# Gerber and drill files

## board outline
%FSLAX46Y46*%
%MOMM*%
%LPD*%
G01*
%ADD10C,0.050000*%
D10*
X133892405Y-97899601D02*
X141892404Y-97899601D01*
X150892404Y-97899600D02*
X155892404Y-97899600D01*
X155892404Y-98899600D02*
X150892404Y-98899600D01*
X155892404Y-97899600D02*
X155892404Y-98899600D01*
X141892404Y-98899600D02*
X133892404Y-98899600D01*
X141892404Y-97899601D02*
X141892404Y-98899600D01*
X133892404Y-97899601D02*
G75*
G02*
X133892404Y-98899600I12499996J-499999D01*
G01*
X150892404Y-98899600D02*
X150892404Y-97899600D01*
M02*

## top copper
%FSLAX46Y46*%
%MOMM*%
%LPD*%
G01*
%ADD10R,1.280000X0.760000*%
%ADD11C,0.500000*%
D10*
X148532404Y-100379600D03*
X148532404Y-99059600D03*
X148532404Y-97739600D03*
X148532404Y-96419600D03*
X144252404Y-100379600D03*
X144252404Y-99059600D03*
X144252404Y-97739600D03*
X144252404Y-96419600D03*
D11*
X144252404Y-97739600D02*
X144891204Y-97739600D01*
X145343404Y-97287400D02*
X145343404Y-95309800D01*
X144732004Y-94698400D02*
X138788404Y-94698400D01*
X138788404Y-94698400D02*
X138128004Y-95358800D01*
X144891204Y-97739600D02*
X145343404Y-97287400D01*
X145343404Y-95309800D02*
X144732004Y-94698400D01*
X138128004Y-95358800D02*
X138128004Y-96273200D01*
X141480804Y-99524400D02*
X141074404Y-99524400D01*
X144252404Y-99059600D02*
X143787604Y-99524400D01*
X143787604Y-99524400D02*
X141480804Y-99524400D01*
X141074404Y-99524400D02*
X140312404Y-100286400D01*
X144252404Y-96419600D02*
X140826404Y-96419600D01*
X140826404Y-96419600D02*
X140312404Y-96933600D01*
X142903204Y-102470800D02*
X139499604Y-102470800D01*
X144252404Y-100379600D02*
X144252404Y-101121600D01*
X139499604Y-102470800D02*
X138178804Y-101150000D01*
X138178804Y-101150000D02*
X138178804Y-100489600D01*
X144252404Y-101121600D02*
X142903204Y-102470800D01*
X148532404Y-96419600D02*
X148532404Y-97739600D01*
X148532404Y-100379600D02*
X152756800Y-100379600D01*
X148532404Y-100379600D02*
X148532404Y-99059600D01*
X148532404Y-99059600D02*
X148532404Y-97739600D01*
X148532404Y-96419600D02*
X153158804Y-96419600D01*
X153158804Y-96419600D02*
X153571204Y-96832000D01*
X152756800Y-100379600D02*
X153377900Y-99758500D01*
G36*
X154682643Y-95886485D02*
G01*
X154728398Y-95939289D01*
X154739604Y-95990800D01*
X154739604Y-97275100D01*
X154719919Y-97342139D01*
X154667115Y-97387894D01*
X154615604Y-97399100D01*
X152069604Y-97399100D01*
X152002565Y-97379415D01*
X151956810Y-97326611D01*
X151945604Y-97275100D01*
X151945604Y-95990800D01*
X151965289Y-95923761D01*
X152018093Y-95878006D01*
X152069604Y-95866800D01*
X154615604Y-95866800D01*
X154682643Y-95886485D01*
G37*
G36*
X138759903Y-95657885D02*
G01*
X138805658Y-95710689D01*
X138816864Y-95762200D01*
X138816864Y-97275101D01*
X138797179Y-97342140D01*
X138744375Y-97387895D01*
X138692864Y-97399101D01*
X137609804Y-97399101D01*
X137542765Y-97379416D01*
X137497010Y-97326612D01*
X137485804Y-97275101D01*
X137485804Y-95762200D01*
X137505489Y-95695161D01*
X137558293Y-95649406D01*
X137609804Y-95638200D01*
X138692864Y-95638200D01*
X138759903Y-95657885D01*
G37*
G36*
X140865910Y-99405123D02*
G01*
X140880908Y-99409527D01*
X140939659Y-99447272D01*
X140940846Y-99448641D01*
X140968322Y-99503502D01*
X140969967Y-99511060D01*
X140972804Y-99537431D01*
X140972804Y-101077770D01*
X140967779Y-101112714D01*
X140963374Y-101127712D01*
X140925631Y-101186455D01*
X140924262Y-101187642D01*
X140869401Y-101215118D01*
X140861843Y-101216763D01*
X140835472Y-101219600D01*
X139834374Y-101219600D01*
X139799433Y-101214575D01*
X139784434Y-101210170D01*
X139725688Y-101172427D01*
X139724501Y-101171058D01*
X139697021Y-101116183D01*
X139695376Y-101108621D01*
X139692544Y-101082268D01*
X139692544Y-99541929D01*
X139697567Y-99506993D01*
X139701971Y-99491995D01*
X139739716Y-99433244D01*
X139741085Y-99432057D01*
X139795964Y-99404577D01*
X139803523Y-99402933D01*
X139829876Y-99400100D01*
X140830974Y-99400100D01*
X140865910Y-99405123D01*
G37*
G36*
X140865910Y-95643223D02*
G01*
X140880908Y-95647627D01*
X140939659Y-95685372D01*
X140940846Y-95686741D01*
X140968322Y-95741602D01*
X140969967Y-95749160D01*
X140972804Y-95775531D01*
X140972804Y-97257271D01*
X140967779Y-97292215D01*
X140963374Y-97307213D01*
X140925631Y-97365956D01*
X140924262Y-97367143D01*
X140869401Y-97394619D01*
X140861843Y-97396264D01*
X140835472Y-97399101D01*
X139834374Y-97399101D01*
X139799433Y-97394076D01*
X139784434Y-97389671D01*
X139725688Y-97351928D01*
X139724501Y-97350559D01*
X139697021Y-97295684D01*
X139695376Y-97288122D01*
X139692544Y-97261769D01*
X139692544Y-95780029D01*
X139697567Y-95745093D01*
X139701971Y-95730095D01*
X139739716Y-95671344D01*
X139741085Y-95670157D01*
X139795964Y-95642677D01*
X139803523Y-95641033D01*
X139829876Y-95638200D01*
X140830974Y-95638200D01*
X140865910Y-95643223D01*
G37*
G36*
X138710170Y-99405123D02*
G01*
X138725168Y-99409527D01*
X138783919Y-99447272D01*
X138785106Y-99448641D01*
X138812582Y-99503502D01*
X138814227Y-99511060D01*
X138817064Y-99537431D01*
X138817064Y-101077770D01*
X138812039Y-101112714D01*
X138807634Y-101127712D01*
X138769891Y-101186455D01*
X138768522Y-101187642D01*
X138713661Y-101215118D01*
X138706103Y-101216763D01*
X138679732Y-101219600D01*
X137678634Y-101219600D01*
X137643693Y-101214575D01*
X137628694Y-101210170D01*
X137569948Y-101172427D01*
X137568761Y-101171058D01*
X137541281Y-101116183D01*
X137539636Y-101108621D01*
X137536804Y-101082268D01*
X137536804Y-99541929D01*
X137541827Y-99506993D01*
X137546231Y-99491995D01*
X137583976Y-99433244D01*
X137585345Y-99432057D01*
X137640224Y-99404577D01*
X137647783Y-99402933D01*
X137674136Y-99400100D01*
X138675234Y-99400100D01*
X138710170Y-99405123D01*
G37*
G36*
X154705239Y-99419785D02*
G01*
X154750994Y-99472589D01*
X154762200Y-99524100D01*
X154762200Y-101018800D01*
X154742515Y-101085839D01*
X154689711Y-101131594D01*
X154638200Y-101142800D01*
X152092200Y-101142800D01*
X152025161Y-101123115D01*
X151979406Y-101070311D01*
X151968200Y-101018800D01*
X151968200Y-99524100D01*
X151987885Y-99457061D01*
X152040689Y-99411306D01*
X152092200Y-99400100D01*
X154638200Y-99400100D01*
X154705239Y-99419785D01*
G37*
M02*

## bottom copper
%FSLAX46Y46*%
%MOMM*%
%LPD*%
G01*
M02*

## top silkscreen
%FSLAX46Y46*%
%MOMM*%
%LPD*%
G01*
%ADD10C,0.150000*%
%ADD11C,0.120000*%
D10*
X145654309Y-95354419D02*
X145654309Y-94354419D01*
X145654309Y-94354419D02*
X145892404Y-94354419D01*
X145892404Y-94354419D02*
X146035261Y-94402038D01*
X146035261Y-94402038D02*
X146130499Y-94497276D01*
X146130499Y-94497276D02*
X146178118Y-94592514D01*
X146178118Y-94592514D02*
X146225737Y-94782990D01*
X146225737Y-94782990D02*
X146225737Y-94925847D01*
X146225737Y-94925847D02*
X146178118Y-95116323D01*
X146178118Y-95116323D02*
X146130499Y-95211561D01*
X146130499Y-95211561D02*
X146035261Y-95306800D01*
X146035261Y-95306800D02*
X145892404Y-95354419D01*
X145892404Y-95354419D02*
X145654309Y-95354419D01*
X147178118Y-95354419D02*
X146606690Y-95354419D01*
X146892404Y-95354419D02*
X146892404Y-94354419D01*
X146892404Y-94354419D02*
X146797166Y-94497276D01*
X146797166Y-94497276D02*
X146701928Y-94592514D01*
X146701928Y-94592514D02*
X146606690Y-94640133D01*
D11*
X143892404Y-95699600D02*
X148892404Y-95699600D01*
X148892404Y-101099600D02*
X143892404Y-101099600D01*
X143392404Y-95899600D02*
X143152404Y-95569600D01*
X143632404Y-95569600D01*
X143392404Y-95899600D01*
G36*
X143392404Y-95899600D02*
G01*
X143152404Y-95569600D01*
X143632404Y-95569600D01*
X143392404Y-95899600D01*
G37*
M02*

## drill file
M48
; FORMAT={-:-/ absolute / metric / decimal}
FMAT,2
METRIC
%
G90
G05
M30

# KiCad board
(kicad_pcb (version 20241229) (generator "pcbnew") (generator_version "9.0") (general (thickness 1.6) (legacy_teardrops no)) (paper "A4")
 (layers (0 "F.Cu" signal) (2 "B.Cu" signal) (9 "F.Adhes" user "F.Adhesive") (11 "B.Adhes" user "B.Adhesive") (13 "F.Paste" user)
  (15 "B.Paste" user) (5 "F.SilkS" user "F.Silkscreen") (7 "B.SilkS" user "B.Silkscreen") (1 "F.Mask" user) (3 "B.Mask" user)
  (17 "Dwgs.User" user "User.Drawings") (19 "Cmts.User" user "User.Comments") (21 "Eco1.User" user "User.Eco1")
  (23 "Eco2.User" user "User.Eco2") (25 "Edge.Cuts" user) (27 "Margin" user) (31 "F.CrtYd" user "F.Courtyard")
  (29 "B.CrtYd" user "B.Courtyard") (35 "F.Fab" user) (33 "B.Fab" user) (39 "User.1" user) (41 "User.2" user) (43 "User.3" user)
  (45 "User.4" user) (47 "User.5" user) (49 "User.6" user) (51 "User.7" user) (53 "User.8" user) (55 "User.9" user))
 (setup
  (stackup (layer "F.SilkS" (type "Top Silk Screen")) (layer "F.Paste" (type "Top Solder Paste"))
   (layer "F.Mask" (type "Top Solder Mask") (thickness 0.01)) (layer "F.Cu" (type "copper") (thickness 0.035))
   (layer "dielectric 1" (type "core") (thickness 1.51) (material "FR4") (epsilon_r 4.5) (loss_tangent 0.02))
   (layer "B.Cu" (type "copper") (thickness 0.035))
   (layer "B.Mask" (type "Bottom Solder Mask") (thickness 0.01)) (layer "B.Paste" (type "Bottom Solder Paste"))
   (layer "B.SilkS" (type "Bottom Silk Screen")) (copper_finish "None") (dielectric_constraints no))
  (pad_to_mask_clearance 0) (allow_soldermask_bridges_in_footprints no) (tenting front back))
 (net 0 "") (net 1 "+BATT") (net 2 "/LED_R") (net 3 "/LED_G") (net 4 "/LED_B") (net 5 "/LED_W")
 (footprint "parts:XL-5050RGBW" (layer "F.Cu") (at 146.392404 98.3996 180)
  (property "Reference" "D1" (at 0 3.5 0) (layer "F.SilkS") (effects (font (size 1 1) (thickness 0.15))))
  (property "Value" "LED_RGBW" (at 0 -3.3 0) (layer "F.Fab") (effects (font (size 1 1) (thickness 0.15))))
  (fp_line (start 2.5 2.7) (end -2.5 2.7) (stroke (width 0.12) (type solid)) (layer "F.SilkS"))
  (fp_line (start -2.5 -2.7) (end 2.5 -2.7) (stroke (width 0.12) (type solid)) (layer "F.SilkS"))
  (fp_poly (pts (xy 3 2.5) (xy 3.24 2.83) (xy 2.76 2.83) (xy 3 2.5)) (stroke (width 0.12) (type solid)) (fill yes) (layer "F.SilkS"))
  (pad "1" smd rect (at -2.14 -1.98 270) (size 0.76 1.28) (layers "F.Cu" "F.Mask" "F.Paste") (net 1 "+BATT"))
  (pad "2" smd rect (at -2.14 -0.66 270) (size 0.76 1.28) (layers "F.Cu" "F.Mask" "F.Paste") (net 1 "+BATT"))
  (pad "3" smd rect (at -2.14 0.66 270) (size 0.76 1.28) (layers "F.Cu" "F.Mask" "F.Paste") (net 1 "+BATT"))
  (pad "4" smd rect (at -2.14 1.98 270) (size 0.76 1.28) (layers "F.Cu" "F.Mask" "F.Paste") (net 1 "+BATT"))
  (pad "5" smd rect (at 2.14 -1.98 270) (size 0.76 1.28) (layers "F.Cu" "F.Mask" "F.Paste") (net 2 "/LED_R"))
  (pad "6" smd rect (at 2.14 -0.66 270) (size 0.76 1.28) (layers "F.Cu" "F.Mask" "F.Paste") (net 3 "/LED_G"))
  (pad "7" smd rect (at 2.14 0.66 270) (size 0.76 1.28) (layers "F.Cu" "F.Mask" "F.Paste") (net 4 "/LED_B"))
  (pad "8" smd rect (at 2.14 1.98 270) (size 0.76 1.28) (layers "F.Cu" "F.Mask" "F.Paste") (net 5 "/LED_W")))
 (gr_line (start 133.892405 97.899601) (end 141.892404 97.899601) (stroke (width 0.05) (type default)) (layer "Edge.Cuts"))
 (gr_line (start 150.892404 97.8996) (end 155.892404 97.8996) (stroke (width 0.05) (type default)) (layer "Edge.Cuts"))
 (gr_line (start 155.892404 98.8996) (end 150.892404 98.8996) (stroke (width 0.05) (type default)) (layer "Edge.Cuts"))
 (gr_line (start 155.892404 97.8996) (end 155.892404 98.8996) (stroke (width 0.05) (type default)) (layer "Edge.Cuts"))
 (gr_line (start 141.892404 98.8996) (end 133.892404 98.8996) (stroke (width 0.05) (type default)) (layer "Edge.Cuts"))
 (gr_line (start 141.892404 97.899601) (end 141.892404 98.8996) (stroke (width 0.05) (type default)) (layer "Edge.Cuts"))
 (gr_arc (start 133.892404 97.899601) (mid 158.9024 98.3996) (end 133.892404 98.8996) (stroke (width 0.05) (type default))
  (layer "Edge.Cuts"))
 (gr_line (start 150.892404 98.8996) (end 150.892404 97.8996) (stroke (width 0.05) (type default)) (layer "Edge.Cuts"))
 (segment (start 144.252404 97.7396) (end 144.891204 97.7396) (width 0.5) (layer "F.Cu") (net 4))
 (segment (start 145.343404 97.2874) (end 145.343404 95.3098) (width 0.5) (layer "F.Cu") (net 4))
 (segment (start 144.732004 94.6984) (end 138.788404 94.6984) (width 0.5) (layer "F.Cu") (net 4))
 (segment (start 138.788404 94.6984) (end 138.128004 95.3588) (width 0.5) (layer "F.Cu") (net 4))
 (segment (start 144.891204 97.7396) (end 145.343404 97.2874) (width 0.5) (layer "F.Cu") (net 4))
 (segment (start 145.343404 95.3098) (end 144.732004 94.6984) (width 0.5) (layer "F.Cu") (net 4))
 (segment (start 138.128004 95.3588) (end 138.128004 96.2732) (width 0.5) (layer "F.Cu") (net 4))
 (segment (start 141.480804 99.5244) (end 141.074404 99.5244) (width 0.5) (layer "F.Cu") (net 3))
 (segment (start 144.252404 99.0596) (end 143.787604 99.5244) (width 0.5) (layer "F.Cu") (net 3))
 (segment (start 143.787604 99.5244) (end 141.480804 99.5244) (width 0.5) (layer "F.Cu") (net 3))
 (segment (start 141.074404 99.5244) (end 140.312404 100.2864) (width 0.5) (layer "F.Cu") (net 3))
 (segment (start 144.252404 96.4196) (end 140.826404 96.4196) (width 0.5) (layer "F.Cu") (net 5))
 (segment (start 140.826404 96.4196) (end 140.312404 96.9336) (width 0.5) (layer "F.Cu") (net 5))
 (segment (start 142.903204 102.4708) (end 139.499604 102.4708) (width 0.5) (layer "F.Cu") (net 2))
 (segment (start 144.252404 100.3796) (end 144.252404 101.1216) (width 0.5) (layer "F.Cu") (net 2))
 (segment (start 139.499604 102.4708) (end 138.178804 101.15) (width 0.5) (layer "F.Cu") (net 2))
 (segment (start 138.178804 101.15) (end 138.178804 100.4896) (width 0.5) (layer "F.Cu") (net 2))
 (segment (start 144.252404 101.1216) (end 142.903204 102.4708) (width 0.5) (layer "F.Cu") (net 2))
 (segment (start 148.532404 96.4196) (end 148.532404 97.7396) (width 0.5) (layer "F.Cu") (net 1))
 (segment (start 148.532404 100.3796) (end 152.7568 100.3796) (width 0.5) (layer "F.Cu") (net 1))
 (segment (start 148.532404 100.3796) (end 148.532404 99.0596) (width 0.5) (layer "F.Cu") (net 1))
 (segment (start 148.532404 99.0596) (end 148.532404 97.7396) (width 0.5) (layer "F.Cu") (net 1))
 (segment (start 148.532404 96.4196) (end 153.158804 96.4196) (width 0.5) (layer "F.Cu") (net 1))
 (segment (start 153.158804 96.4196) (end 153.571204 96.832) (width 0.5) (layer "F.Cu") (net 1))
 (segment (start 152.7568 100.3796) (end 153.3779 99.7585) (width 0.5) (layer "F.Cu") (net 1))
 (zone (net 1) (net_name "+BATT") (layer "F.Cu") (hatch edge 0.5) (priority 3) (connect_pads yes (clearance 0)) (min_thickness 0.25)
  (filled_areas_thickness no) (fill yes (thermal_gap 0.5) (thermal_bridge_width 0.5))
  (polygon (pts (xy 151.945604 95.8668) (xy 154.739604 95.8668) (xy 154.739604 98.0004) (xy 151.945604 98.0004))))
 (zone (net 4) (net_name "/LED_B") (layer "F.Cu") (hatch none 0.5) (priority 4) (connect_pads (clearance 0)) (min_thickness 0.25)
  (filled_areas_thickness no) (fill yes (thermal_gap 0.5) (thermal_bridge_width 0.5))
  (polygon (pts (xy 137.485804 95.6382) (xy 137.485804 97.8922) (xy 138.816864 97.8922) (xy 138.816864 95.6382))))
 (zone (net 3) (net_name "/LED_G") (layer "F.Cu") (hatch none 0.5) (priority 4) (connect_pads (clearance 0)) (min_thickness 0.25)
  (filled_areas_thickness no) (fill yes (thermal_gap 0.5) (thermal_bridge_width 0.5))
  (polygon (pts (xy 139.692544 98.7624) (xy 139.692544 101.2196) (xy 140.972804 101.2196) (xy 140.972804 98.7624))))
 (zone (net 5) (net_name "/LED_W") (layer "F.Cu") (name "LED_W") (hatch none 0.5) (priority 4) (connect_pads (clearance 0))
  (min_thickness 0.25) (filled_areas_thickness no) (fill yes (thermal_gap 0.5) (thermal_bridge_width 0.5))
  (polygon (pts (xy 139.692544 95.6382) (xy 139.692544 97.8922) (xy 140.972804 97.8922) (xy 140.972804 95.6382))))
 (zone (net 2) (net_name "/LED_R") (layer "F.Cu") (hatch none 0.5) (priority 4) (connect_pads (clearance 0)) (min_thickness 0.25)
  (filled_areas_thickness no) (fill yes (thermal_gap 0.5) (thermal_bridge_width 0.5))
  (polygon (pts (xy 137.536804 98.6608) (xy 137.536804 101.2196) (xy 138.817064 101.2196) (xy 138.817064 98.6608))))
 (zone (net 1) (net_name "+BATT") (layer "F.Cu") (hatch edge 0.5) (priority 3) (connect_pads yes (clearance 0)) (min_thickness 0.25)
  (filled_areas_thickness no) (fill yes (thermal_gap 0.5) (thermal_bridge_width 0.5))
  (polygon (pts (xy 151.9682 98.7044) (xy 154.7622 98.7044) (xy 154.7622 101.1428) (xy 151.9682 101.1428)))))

